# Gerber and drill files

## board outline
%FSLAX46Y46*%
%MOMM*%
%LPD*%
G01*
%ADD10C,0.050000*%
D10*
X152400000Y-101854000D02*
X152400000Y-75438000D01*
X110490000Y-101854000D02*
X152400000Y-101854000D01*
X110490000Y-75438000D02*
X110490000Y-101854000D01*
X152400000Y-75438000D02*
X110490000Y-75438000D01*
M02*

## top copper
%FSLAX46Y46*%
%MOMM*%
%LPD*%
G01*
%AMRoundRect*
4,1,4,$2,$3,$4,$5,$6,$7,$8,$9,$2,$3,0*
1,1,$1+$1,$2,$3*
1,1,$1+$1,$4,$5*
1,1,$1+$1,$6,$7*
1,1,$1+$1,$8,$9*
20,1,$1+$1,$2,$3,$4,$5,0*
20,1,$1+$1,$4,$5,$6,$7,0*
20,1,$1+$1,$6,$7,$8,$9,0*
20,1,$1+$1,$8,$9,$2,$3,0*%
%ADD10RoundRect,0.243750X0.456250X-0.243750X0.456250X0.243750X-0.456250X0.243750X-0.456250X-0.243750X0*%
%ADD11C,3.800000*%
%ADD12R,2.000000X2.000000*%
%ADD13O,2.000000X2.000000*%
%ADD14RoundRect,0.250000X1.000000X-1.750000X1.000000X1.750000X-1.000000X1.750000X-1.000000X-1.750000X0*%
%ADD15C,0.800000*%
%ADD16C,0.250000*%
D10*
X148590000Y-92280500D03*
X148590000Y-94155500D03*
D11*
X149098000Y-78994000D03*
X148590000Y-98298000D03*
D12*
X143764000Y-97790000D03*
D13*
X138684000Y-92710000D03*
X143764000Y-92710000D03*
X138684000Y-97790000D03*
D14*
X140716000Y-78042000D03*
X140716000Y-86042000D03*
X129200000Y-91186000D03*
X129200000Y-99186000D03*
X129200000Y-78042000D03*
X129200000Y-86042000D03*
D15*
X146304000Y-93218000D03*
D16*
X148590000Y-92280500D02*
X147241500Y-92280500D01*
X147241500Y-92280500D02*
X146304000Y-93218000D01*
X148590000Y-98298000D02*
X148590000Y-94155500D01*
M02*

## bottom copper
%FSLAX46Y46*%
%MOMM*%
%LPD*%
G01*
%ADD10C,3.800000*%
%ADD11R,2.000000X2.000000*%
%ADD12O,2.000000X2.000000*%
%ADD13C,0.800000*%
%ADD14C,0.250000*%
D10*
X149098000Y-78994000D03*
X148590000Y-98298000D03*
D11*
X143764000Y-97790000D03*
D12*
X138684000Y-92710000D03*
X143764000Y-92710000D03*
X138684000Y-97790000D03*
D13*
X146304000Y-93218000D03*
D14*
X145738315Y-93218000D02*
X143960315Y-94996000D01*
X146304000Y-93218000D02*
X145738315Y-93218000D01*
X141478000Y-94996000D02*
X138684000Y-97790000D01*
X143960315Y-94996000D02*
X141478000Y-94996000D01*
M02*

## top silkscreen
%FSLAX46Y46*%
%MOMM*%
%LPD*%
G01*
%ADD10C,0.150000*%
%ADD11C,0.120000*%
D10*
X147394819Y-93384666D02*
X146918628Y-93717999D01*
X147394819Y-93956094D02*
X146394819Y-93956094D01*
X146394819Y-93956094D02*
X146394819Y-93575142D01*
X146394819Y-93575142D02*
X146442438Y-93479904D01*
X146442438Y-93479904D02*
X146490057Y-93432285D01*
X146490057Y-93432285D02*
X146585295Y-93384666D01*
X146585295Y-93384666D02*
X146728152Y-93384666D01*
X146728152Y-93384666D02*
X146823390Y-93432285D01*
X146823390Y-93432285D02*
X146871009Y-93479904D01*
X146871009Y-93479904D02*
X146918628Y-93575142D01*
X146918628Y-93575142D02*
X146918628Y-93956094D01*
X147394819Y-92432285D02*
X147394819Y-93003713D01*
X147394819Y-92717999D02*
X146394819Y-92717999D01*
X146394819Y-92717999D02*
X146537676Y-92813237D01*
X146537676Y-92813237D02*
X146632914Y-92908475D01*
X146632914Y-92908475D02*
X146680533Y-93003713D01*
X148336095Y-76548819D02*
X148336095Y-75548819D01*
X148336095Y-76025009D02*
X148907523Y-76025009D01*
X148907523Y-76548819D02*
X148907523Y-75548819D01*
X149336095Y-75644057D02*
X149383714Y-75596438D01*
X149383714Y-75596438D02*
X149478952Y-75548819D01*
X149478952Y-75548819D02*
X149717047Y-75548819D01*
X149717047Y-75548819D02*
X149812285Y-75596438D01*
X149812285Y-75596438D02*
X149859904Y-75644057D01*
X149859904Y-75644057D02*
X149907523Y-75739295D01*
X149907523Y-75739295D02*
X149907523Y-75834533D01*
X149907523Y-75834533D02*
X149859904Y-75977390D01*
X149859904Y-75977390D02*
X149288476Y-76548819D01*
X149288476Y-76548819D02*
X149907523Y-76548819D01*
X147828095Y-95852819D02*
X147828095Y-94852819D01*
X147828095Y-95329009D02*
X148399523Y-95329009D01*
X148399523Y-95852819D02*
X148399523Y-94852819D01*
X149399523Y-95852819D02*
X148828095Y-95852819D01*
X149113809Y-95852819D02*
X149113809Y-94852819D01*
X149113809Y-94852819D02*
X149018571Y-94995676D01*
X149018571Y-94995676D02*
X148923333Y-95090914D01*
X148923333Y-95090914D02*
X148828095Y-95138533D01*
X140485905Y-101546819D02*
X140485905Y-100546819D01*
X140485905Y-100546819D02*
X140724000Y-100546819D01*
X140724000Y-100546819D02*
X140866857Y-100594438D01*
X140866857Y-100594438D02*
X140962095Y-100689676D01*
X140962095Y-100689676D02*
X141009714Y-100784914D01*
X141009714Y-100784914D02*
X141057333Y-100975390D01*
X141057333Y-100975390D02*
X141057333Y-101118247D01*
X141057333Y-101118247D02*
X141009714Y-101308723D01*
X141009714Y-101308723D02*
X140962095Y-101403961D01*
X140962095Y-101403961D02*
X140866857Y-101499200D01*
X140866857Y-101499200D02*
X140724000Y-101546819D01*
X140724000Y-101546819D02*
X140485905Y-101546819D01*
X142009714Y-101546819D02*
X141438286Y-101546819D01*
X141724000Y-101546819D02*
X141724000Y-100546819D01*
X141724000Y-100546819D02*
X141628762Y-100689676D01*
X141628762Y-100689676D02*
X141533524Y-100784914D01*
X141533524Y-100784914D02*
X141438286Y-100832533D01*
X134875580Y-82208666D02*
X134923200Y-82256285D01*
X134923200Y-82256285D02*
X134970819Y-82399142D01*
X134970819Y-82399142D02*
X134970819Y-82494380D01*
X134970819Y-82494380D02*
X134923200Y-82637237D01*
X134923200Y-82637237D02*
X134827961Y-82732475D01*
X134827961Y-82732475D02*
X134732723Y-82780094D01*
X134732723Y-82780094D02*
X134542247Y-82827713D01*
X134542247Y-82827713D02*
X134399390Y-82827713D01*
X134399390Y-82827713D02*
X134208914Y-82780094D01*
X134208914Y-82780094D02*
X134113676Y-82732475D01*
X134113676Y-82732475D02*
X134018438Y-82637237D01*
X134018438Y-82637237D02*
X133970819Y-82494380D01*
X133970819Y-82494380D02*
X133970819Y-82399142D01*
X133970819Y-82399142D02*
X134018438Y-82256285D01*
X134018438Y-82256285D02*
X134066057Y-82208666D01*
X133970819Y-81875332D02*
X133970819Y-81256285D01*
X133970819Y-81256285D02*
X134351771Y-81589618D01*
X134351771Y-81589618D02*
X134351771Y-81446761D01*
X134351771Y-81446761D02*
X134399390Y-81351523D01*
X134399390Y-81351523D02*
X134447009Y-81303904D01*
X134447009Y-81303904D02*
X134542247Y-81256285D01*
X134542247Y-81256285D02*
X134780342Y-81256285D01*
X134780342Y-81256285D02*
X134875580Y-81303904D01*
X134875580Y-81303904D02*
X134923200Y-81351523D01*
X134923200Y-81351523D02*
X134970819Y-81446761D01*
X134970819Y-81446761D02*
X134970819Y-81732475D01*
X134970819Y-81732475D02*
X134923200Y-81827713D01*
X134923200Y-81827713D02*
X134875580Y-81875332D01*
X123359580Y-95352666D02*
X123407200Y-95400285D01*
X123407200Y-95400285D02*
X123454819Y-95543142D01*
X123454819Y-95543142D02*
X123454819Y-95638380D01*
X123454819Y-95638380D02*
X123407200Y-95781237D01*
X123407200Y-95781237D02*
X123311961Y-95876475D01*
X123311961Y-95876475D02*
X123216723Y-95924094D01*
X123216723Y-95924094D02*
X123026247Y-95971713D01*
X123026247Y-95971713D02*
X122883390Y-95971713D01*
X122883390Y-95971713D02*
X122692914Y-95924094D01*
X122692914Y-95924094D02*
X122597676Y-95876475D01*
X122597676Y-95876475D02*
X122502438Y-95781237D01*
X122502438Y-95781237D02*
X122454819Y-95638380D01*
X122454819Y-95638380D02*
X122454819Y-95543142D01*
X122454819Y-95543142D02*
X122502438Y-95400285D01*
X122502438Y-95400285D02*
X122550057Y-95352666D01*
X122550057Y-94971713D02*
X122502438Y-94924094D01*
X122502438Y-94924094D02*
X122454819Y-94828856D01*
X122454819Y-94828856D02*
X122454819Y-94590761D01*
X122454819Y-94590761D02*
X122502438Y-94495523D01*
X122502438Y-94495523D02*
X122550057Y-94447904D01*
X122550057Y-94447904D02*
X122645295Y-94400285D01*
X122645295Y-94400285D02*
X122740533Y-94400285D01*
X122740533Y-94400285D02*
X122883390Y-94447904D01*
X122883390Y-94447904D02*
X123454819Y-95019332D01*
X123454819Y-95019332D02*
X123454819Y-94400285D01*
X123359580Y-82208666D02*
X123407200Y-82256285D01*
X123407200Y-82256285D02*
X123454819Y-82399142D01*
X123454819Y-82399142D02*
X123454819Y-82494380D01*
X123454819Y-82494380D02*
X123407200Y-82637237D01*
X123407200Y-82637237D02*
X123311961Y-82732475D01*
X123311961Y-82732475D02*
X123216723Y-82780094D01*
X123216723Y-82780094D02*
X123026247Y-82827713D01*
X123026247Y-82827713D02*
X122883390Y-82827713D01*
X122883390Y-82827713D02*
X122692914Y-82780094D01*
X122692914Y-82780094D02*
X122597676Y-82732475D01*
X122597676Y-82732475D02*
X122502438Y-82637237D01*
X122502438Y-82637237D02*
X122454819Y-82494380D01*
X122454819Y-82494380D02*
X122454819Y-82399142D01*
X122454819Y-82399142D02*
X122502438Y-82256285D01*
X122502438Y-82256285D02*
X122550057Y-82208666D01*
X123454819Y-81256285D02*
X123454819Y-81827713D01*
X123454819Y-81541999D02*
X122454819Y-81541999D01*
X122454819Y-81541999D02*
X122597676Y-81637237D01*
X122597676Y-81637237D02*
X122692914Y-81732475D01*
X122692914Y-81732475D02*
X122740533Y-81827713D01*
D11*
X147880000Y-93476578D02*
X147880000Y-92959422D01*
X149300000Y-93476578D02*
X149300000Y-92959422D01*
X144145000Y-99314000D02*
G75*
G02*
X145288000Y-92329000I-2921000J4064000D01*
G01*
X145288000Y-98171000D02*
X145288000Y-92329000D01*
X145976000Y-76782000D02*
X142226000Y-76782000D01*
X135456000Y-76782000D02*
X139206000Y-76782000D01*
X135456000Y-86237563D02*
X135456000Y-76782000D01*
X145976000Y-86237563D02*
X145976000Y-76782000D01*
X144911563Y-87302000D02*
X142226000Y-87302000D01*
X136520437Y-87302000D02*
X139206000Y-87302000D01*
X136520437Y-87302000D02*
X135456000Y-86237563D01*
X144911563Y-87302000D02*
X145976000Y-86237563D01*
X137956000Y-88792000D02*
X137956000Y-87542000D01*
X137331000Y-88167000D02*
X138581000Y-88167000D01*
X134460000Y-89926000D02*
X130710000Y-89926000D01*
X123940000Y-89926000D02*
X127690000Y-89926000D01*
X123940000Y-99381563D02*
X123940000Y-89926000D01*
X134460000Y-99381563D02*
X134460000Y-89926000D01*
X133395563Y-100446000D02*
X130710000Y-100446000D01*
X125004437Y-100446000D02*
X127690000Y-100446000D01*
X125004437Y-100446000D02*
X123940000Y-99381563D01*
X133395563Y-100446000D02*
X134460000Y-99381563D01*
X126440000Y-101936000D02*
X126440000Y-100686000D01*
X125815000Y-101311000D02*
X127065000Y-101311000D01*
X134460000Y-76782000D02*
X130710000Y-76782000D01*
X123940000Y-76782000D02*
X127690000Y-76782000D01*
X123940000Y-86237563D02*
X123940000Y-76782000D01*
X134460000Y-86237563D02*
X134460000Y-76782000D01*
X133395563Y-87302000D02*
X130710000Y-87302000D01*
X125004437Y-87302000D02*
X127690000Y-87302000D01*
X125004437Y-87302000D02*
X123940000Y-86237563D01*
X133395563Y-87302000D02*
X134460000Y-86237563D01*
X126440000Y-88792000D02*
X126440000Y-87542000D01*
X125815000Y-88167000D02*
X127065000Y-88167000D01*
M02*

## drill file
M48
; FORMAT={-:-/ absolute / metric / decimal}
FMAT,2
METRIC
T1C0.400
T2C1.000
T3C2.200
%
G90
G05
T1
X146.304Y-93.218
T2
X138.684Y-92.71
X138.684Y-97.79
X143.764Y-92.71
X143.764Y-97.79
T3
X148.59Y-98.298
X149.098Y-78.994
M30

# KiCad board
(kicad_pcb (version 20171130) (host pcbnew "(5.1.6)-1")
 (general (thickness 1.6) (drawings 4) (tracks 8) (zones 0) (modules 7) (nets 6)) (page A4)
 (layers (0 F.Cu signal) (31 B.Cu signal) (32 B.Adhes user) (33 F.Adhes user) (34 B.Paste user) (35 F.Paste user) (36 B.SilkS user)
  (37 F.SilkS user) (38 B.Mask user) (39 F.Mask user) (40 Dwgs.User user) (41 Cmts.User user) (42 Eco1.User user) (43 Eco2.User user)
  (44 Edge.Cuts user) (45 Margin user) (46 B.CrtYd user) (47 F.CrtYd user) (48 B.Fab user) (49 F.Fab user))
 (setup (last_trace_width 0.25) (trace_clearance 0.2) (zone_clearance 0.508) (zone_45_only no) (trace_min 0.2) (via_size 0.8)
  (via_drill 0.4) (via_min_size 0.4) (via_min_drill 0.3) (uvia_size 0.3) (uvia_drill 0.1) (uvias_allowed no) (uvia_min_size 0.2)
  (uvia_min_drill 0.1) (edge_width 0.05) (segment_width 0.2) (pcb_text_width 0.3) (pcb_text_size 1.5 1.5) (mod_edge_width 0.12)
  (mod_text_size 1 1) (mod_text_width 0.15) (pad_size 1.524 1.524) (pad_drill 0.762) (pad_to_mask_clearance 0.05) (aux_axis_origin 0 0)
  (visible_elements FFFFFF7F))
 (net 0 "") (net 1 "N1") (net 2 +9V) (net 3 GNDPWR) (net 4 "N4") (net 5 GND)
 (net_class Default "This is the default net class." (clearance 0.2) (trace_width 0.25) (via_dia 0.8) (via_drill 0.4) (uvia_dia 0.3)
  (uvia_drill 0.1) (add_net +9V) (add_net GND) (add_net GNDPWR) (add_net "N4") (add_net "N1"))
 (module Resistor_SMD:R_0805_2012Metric (layer F.Cu) (at 148.59 93.218 90)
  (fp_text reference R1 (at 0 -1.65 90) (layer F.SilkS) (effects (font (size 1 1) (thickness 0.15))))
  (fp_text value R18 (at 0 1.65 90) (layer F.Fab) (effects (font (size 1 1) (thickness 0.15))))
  (fp_line (start -0.258578 -0.71) (end 0.258578 -0.71) (layer F.SilkS) (width 0.12))
  (fp_line (start -0.258578 0.71) (end 0.258578 0.71) (layer F.SilkS) (width 0.12))
  (pad 2 smd roundrect (at 0.9375 0 90) (size 0.975 1.4) (layers F.Cu F.Paste F.Mask) (roundrect_rratio 0.25) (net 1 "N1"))
  (pad 1 smd roundrect (at -0.9375 0 90) (size 0.975 1.4) (layers F.Cu F.Paste F.Mask) (roundrect_rratio 0.25) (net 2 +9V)))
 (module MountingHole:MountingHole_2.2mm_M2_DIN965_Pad (layer F.Cu) (at 149.098 78.994)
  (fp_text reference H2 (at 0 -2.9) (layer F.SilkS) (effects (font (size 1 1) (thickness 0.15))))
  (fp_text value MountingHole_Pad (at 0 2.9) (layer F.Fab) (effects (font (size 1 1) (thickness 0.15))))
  (pad 1 thru_hole circle (at 0 0) (size 3.8 3.8) (drill 2.2) (layers *.Cu *.Mask) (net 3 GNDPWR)))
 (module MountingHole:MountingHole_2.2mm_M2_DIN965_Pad (layer F.Cu) (at 148.59 98.298)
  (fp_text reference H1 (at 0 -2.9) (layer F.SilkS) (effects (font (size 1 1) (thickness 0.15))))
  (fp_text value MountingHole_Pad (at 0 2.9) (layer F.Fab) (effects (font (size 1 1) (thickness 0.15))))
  (pad 1 thru_hole circle (at 0 0) (size 3.8 3.8) (drill 2.2) (layers *.Cu *.Mask) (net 2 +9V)))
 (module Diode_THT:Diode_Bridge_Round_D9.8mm (layer F.Cu) (at 143.764 97.79 180)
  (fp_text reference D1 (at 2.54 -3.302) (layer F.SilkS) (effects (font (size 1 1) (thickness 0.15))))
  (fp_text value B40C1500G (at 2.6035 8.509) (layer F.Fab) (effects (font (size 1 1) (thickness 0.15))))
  (fp_arc (start 2.54 2.54) (end -0.381 -1.524) (angle 270) (layer F.SilkS) (width 0.12))
  (fp_line (start -1.524 -0.381) (end -1.524 5.461) (layer F.SilkS) (width 0.12))
  (pad 1 thru_hole rect (at 0 0 180) (size 2 2) (drill 1) (layers *.Cu *.Mask) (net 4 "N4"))
  (pad 3 thru_hole oval (at 5.08 5.08 180) (size 2 2) (drill 1) (layers *.Cu *.Mask) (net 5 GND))
  (pad 2 thru_hole oval (at 0 5.08 180) (size 2 2) (drill 1) (layers *.Cu *.Mask) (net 3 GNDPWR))
  (pad 4 thru_hole oval (at 5.08 0 180) (size 2 2) (drill 1) (layers *.Cu *.Mask) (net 1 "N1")))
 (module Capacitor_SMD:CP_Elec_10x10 (layer F.Cu) (at 140.716 82.042 90)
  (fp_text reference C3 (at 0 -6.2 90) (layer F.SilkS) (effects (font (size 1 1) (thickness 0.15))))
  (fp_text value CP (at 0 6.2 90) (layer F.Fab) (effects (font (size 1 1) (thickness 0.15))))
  (fp_line (start 5.26 5.26) (end 5.26 1.51) (layer F.SilkS) (width 0.12))
  (fp_line (start 5.26 -5.26) (end 5.26 -1.51) (layer F.SilkS) (width 0.12))
  (fp_line (start -4.195563 -5.26) (end 5.26 -5.26) (layer F.SilkS) (width 0.12))
  (fp_line (start -4.195563 5.26) (end 5.26 5.26) (layer F.SilkS) (width 0.12))
  (fp_line (start -5.26 4.195563) (end -5.26 1.51) (layer F.SilkS) (width 0.12))
  (fp_line (start -5.26 -4.195563) (end -5.26 -1.51) (layer F.SilkS) (width 0.12))
  (fp_line (start -5.26 -4.195563) (end -4.195563 -5.26) (layer F.SilkS) (width 0.12))
  (fp_line (start -5.26 4.195563) (end -4.195563 5.26) (layer F.SilkS) (width 0.12))
  (fp_line (start -6.75 -2.76) (end -5.5 -2.76) (layer F.SilkS) (width 0.12))
  (fp_line (start -6.125 -3.385) (end -6.125 -2.135) (layer F.SilkS) (width 0.12))
  (pad 2 smd roundrect (at 4 0 90) (size 4 2.5) (layers F.Cu F.Paste F.Mask) (roundrect_rratio 0.1) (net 5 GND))
  (pad 1 smd roundrect (at -4 0 90) (size 4 2.5) (layers F.Cu F.Paste F.Mask) (roundrect_rratio 0.1) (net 4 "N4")))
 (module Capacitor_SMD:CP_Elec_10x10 (layer F.Cu) (at 129.2 95.186 90)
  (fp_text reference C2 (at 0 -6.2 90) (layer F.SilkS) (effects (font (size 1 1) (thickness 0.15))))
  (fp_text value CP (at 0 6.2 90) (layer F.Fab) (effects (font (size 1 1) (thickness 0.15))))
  (fp_line (start 5.26 5.26) (end 5.26 1.51) (layer F.SilkS) (width 0.12))
  (fp_line (start 5.26 -5.26) (end 5.26 -1.51) (layer F.SilkS) (width 0.12))
  (fp_line (start -4.195563 -5.26) (end 5.26 -5.26) (layer F.SilkS) (width 0.12))
  (fp_line (start -4.195563 5.26) (end 5.26 5.26) (layer F.SilkS) (width 0.12))
  (fp_line (start -5.26 4.195563) (end -5.26 1.51) (layer F.SilkS) (width 0.12))
  (fp_line (start -5.26 -4.195563) (end -5.26 -1.51) (layer F.SilkS) (width 0.12))
  (fp_line (start -5.26 -4.195563) (end -4.195563 -5.26) (layer F.SilkS) (width 0.12))
  (fp_line (start -5.26 4.195563) (end -4.195563 5.26) (layer F.SilkS) (width 0.12))
  (fp_line (start -6.75 -2.76) (end -5.5 -2.76) (layer F.SilkS) (width 0.12))
  (fp_line (start -6.125 -3.385) (end -6.125 -2.135) (layer F.SilkS) (width 0.12))
  (pad 2 smd roundrect (at 4 0 90) (size 4 2.5) (layers F.Cu F.Paste F.Mask) (roundrect_rratio 0.1) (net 5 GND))
  (pad 1 smd roundrect (at -4 0 90) (size 4 2.5) (layers F.Cu F.Paste F.Mask) (roundrect_rratio 0.1) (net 4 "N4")))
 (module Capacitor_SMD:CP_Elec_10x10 (layer F.Cu) (at 129.2 82.042 90)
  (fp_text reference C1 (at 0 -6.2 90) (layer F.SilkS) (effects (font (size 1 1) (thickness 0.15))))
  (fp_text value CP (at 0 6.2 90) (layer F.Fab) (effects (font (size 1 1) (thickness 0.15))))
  (fp_line (start 5.26 5.26) (end 5.26 1.51) (layer F.SilkS) (width 0.12))
  (fp_line (start 5.26 -5.26) (end 5.26 -1.51) (layer F.SilkS) (width 0.12))
  (fp_line (start -4.195563 -5.26) (end 5.26 -5.26) (layer F.SilkS) (width 0.12))
  (fp_line (start -4.195563 5.26) (end 5.26 5.26) (layer F.SilkS) (width 0.12))
  (fp_line (start -5.26 4.195563) (end -5.26 1.51) (layer F.SilkS) (width 0.12))
  (fp_line (start -5.26 -4.195563) (end -5.26 -1.51) (layer F.SilkS) (width 0.12))
  (fp_line (start -5.26 -4.195563) (end -4.195563 -5.26) (layer F.SilkS) (width 0.12))
  (fp_line (start -5.26 4.195563) (end -4.195563 5.26) (layer F.SilkS) (width 0.12))
  (fp_line (start -6.75 -2.76) (end -5.5 -2.76) (layer F.SilkS) (width 0.12))
  (fp_line (start -6.125 -3.385) (end -6.125 -2.135) (layer F.SilkS) (width 0.12))
  (pad 2 smd roundrect (at 4 0 90) (size 4 2.5) (layers F.Cu F.Paste F.Mask) (roundrect_rratio 0.1) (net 5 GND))
  (pad 1 smd roundrect (at -4 0 90) (size 4 2.5) (layers F.Cu F.Paste F.Mask) (roundrect_rratio 0.1) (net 4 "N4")))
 (gr_line (start 152.4 101.854) (end 152.4 75.438) (layer Edge.Cuts) (width 0.05))
 (gr_line (start 110.49 101.854) (end 152.4 101.854) (layer Edge.Cuts) (width 0.05))
 (gr_line (start 110.49 75.438) (end 110.49 101.854) (layer Edge.Cuts) (width 0.05))
 (gr_line (start 152.4 75.438) (end 110.49 75.438) (layer Edge.Cuts) (width 0.05))
 (via (at 146.304 93.218) (size 0.8) (drill 0.4) (layers F.Cu B.Cu) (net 1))
 (segment (start 148.59 92.2805) (end 147.2415 92.2805) (width 0.25) (layer F.Cu) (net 1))
 (segment (start 147.2415 92.2805) (end 146.304 93.218) (width 0.25) (layer F.Cu) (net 1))
 (segment (start 145.738315 93.218) (end 143.960315 94.996) (width 0.25) (layer B.Cu) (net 1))
 (segment (start 146.304 93.218) (end 145.738315 93.218) (width 0.25) (layer B.Cu) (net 1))
 (segment (start 141.478 94.996) (end 138.684 97.79) (width 0.25) (layer B.Cu) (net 1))
 (segment (start 143.960315 94.996) (end 141.478 94.996) (width 0.25) (layer B.Cu) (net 1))
 (segment (start 148.59 98.298) (end 148.59 94.1555) (width 0.25) (layer F.Cu) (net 2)))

